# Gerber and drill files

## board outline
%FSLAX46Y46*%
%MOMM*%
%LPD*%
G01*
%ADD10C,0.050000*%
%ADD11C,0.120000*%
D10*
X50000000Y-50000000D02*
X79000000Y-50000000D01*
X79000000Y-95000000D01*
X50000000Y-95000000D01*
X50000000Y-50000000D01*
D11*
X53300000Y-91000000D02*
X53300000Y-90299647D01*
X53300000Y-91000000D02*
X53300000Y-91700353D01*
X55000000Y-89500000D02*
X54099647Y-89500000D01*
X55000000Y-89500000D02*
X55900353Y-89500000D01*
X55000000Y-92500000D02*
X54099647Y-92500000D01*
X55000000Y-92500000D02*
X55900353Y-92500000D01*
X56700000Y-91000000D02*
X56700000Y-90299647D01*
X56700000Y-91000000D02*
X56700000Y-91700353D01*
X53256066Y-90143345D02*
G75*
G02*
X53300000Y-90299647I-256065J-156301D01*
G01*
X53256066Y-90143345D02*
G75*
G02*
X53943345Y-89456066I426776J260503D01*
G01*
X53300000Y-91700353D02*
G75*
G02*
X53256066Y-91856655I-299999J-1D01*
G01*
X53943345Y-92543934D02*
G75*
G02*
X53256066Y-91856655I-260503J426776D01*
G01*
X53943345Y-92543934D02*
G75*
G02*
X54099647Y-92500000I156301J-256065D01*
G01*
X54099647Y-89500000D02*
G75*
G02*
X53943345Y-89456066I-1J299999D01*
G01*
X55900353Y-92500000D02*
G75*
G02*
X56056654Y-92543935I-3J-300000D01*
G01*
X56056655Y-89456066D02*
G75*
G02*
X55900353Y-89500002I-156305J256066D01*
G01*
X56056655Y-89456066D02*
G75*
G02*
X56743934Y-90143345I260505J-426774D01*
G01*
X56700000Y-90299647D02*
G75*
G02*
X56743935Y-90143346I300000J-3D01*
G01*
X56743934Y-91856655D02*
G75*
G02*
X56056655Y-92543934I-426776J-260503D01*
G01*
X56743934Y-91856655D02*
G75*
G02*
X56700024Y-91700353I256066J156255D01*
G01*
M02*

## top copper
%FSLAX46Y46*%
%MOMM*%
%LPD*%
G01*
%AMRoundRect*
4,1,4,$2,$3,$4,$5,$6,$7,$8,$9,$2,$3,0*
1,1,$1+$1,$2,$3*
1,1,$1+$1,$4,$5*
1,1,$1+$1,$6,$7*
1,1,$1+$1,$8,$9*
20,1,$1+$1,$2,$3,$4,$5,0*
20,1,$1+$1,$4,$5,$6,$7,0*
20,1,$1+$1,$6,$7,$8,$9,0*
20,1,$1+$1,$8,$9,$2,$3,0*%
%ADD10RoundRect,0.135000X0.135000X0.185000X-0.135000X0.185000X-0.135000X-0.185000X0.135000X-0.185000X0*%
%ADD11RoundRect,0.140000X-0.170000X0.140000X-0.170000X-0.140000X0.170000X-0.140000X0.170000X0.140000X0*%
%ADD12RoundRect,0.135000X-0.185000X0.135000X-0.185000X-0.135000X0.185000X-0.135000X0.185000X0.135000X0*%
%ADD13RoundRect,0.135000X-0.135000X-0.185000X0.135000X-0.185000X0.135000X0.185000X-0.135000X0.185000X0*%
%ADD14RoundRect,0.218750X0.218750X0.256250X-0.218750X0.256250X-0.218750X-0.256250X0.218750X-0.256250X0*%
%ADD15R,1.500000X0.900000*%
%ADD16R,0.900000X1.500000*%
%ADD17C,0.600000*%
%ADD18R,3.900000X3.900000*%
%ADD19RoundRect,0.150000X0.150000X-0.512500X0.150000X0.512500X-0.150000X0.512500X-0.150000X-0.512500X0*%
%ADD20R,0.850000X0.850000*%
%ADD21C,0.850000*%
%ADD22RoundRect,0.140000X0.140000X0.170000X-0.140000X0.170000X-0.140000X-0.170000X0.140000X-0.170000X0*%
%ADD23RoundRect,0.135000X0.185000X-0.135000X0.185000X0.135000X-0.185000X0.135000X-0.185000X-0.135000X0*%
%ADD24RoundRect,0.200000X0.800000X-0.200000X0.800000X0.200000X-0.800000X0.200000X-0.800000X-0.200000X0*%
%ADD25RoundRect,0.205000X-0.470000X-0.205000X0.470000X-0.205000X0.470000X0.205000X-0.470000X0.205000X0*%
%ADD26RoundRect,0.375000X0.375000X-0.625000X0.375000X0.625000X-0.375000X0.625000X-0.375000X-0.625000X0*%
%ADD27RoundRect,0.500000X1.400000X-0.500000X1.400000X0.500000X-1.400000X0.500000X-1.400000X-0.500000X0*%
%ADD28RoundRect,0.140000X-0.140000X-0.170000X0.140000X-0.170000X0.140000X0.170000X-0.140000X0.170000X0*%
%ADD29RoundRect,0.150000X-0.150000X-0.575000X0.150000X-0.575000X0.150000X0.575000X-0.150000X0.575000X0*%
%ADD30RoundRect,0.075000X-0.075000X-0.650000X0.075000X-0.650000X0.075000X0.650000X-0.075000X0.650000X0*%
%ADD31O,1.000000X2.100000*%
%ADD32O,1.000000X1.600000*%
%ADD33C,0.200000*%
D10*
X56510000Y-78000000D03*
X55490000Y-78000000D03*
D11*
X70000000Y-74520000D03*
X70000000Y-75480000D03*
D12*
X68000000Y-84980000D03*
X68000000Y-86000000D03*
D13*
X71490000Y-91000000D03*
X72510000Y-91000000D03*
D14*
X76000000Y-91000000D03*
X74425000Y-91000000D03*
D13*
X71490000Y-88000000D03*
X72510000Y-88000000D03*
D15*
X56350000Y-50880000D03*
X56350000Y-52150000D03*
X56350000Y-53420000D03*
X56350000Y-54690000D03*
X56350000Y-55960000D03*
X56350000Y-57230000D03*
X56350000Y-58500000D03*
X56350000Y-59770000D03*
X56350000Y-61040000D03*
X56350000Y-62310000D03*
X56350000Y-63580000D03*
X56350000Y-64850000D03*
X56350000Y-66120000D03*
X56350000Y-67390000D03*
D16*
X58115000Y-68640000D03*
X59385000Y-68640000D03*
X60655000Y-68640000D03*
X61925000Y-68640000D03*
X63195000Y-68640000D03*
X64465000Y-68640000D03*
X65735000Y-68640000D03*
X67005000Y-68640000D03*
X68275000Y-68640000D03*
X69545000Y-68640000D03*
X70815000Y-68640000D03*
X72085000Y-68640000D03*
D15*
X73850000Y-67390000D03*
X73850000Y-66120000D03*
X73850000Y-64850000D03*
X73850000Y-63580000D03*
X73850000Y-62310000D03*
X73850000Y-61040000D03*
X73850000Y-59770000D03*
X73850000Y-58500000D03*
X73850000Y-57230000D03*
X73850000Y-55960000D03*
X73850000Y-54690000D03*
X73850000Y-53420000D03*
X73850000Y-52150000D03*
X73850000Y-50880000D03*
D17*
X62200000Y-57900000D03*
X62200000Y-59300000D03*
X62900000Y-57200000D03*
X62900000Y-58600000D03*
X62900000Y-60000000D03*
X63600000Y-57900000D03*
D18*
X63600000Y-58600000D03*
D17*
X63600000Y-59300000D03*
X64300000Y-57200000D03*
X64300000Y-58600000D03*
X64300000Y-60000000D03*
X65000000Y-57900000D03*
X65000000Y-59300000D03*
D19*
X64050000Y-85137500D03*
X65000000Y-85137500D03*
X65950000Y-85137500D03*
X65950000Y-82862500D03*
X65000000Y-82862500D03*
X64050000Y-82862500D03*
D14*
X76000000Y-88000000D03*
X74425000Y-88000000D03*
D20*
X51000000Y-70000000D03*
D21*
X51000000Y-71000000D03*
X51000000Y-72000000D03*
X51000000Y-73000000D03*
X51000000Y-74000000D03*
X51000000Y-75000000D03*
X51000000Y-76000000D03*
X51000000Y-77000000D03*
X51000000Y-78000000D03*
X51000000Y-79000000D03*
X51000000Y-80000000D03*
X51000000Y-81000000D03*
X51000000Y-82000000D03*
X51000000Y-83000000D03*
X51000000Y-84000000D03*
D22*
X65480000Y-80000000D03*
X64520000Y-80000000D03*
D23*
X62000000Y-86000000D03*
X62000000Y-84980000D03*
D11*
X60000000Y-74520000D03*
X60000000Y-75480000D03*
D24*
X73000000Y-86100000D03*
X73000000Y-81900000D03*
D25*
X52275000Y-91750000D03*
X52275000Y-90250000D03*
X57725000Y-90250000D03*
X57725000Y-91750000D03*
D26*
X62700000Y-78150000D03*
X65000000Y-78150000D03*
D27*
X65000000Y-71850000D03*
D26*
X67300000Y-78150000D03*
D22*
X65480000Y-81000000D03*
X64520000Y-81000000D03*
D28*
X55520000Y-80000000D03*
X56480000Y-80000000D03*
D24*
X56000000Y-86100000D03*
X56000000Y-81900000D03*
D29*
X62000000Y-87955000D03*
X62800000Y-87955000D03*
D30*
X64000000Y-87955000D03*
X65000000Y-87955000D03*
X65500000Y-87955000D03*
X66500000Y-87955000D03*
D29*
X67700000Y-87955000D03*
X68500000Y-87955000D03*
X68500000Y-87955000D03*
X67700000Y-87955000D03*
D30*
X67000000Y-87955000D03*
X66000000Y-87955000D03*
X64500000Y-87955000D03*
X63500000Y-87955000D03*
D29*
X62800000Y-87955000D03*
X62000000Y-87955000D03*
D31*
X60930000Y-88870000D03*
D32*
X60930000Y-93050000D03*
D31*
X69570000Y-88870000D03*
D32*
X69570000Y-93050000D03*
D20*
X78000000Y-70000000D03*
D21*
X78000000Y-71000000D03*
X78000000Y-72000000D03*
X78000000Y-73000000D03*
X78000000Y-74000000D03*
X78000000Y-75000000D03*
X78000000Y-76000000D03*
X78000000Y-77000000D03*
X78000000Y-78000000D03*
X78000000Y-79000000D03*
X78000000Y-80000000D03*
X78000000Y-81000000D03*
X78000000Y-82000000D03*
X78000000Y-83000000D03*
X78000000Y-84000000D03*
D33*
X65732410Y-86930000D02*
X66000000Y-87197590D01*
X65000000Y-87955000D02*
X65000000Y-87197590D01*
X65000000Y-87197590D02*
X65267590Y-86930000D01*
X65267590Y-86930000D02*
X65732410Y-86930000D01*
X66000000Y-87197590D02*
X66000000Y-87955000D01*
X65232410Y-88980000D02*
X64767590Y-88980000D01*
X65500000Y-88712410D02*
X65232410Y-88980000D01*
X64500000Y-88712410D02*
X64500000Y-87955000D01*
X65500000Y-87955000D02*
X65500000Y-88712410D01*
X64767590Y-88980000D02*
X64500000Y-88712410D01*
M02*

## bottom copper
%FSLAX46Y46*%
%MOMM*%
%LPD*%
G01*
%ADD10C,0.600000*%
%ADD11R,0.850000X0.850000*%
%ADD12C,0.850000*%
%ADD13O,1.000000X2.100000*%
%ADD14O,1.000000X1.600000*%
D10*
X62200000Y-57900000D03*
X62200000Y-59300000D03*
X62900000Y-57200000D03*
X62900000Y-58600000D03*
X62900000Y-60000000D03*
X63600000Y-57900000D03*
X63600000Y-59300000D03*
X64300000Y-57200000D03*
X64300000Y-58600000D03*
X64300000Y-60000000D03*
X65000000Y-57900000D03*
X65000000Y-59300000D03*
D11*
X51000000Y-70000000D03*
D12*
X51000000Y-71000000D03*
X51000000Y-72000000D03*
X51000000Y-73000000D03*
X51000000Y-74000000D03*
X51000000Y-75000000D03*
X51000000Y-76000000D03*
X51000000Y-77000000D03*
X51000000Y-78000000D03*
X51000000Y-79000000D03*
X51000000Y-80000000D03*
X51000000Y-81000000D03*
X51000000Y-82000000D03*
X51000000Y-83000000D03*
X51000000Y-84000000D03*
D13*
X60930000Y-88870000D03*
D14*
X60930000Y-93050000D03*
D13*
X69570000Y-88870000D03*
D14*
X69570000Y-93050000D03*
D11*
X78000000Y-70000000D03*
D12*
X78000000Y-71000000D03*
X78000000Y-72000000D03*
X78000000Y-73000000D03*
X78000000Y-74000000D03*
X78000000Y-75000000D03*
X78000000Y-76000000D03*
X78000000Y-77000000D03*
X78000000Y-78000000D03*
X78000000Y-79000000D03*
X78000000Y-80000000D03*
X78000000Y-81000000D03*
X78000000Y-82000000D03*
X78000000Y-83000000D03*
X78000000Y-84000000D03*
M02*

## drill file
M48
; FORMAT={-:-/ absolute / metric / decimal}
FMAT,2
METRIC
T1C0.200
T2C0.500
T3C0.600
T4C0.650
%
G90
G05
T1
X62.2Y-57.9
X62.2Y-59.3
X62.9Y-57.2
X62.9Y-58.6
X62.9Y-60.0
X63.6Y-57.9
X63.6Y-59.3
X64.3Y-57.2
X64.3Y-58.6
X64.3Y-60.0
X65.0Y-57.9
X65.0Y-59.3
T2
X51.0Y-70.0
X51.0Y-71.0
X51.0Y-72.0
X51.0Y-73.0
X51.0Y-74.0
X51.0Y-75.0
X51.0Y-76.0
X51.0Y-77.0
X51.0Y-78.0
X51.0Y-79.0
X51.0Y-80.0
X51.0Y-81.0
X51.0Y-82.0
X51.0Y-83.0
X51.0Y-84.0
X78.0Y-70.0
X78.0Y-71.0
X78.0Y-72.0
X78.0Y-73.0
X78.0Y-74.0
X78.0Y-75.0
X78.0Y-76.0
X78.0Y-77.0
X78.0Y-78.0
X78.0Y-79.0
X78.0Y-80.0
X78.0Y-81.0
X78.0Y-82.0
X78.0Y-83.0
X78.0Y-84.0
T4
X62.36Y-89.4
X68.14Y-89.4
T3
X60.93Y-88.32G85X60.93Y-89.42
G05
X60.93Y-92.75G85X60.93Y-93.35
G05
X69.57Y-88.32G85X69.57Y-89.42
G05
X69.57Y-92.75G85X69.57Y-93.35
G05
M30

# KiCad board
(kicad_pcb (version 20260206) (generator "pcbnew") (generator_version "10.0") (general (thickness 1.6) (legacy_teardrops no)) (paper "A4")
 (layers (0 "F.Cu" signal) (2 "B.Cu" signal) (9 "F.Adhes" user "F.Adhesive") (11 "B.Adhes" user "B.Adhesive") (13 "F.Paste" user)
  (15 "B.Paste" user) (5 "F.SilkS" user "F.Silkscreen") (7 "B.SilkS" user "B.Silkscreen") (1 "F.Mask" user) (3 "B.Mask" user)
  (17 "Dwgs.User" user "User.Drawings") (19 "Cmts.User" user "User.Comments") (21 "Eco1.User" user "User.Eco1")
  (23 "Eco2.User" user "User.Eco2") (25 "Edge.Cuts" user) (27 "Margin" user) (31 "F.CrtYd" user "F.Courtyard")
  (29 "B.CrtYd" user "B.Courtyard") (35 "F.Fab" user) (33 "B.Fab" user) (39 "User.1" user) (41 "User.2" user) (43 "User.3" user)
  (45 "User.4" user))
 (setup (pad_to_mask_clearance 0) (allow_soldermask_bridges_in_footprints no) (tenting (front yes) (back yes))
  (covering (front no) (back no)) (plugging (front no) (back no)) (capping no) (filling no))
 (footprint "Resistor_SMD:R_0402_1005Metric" (layer "F.Cu") (at 56 78 180)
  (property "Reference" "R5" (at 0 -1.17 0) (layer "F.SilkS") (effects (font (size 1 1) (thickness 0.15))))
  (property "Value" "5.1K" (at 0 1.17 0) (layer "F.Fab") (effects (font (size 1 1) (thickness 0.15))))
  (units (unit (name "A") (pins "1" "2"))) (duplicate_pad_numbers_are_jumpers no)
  (pad "1" smd roundrect (at -0.51 0 180) (size 0.54 0.64) (layers "F.Cu" "F.Mask" "F.Paste") (roundrect_rratio 0.25) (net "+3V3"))
  (pad "2" smd roundrect (at 0.51 0 180) (size 0.54 0.64) (layers "F.Cu" "F.Mask" "F.Paste") (roundrect_rratio 0.25) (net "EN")))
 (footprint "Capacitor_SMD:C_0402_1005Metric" (layer "F.Cu") (at 70 75 -90)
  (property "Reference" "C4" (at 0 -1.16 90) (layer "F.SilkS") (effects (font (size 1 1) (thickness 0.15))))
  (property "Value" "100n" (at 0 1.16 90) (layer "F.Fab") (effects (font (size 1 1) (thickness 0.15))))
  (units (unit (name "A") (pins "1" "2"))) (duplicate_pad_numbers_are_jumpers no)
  (pad "1" smd roundrect (at -0.48 0 270) (size 0.56 0.62) (layers "F.Cu" "F.Mask" "F.Paste") (roundrect_rratio 0.25) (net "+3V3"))
  (pad "2" smd roundrect (at 0.48 0 270) (size 0.56 0.62) (layers "F.Cu" "F.Mask" "F.Paste") (roundrect_rratio 0.25) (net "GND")))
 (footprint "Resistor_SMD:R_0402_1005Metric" (layer "F.Cu") (at 68 85.49 -90)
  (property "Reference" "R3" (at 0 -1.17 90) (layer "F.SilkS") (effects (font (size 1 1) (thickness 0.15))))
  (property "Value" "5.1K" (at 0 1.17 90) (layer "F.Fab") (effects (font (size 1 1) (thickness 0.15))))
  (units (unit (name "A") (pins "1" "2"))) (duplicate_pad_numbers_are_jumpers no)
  (pad "1" smd roundrect (at -0.51 0 270) (size 0.54 0.64) (layers "F.Cu" "F.Mask" "F.Paste") (roundrect_rratio 0.25) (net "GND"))
  (pad "2" smd roundrect (at 0.51 0 270) (size 0.54 0.64) (layers "F.Cu" "F.Mask" "F.Paste") (roundrect_rratio 0.25) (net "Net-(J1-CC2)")))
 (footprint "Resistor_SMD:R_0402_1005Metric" (layer "F.Cu") (at 72 91)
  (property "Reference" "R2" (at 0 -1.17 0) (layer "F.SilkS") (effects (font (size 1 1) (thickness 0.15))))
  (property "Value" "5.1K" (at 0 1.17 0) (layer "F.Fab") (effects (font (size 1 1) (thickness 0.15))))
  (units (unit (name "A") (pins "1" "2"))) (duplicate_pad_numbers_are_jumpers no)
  (pad "1" smd roundrect (at -0.51 0) (size 0.54 0.64) (layers "F.Cu" "F.Mask" "F.Paste") (roundrect_rratio 0.25) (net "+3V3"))
  (pad "2" smd roundrect (at 0.51 0) (size 0.54 0.64) (layers "F.Cu" "F.Mask" "F.Paste") (roundrect_rratio 0.25) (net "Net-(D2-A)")))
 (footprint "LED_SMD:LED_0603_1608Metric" (layer "F.Cu") (at 75.2125 91 180)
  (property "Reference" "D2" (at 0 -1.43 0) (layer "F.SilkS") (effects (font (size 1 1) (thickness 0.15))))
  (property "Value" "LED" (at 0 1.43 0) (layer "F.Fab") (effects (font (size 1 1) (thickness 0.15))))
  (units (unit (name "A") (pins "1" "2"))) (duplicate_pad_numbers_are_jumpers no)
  (pad "1" smd roundrect (at -0.7875 0 180) (size 0.875 0.95) (layers "F.Cu" "F.Mask" "F.Paste") (roundrect_rratio 0.25) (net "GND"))
  (pad "2" smd roundrect (at 0.7875 0 180) (size 0.875 0.95) (layers "F.Cu" "F.Mask" "F.Paste") (roundrect_rratio 0.25) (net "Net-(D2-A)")))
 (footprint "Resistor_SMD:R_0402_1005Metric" (layer "F.Cu") (at 72 88)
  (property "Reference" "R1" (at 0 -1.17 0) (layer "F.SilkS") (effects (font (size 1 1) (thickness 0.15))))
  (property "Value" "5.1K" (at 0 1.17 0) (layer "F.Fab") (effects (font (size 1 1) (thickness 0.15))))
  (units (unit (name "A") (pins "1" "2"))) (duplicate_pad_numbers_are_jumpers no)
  (pad "1" smd roundrect (at -0.51 0) (size 0.54 0.64) (layers "F.Cu" "F.Mask" "F.Paste") (roundrect_rratio 0.25) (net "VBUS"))
  (pad "2" smd roundrect (at 0.51 0) (size 0.54 0.64) (layers "F.Cu" "F.Mask" "F.Paste") (roundrect_rratio 0.25) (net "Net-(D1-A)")))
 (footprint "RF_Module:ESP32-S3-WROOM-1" (layer "F.Cu") (at 65.1 56.14)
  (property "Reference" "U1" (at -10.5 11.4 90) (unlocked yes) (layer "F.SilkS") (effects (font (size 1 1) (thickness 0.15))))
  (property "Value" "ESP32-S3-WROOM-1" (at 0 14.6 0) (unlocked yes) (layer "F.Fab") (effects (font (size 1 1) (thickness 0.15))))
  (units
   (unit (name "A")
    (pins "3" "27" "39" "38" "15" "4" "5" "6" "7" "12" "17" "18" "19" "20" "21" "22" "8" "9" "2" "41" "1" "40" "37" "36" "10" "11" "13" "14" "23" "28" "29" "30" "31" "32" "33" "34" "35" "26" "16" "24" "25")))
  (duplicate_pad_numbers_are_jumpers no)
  (pad "" smd rect (at -2.9 1.06) (size 0.9 0.9) (layers "F.Paste"))
  (pad "" smd rect (at -2.9 2.46 270) (size 0.9 0.9) (layers "F.Paste"))
  (pad "" smd rect (at -2.9 3.86) (size 0.9 0.9) (layers "F.Paste"))
  (pad "" smd rect (at -1.5 1.06 270) (size 0.9 0.9) (layers "F.Paste"))
  (pad "" smd rect (at -1.5 2.46 270) (size 0.9 0.9) (layers "F.Paste"))
  (pad "" smd rect (at -1.5 3.86 270) (size 0.9 0.9) (layers "F.Paste"))
  (pad "" smd rect (at -0.1 1.06 270) (size 0.9 0.9) (layers "F.Paste"))
  (pad "" smd rect (at -0.1 2.46 270) (size 0.9 0.9) (layers "F.Paste"))
  (pad "" smd rect (at -0.1 3.86 270) (size 0.9 0.9) (layers "F.Paste"))
  (pad "1" smd rect (at -8.75 -5.26) (size 1.5 0.9) (layers "F.Cu" "F.Mask" "F.Paste") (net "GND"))
  (pad "2" smd rect (at -8.75 -3.99) (size 1.5 0.9) (layers "F.Cu" "F.Mask" "F.Paste") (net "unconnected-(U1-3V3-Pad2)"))
  (pad "3" smd rect (at -8.75 -2.72) (size 1.5 0.9) (layers "F.Cu" "F.Mask" "F.Paste") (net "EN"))
  (pad "4" smd rect (at -8.75 -1.45) (size 1.5 0.9) (layers "F.Cu" "F.Mask" "F.Paste") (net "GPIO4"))
  (pad "5" smd rect (at -8.75 -0.18) (size 1.5 0.9) (layers "F.Cu" "F.Mask" "F.Paste") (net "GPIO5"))
  (pad "6" smd rect (at -8.75 1.09) (size 1.5 0.9) (layers "F.Cu" "F.Mask" "F.Paste") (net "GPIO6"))
  (pad "7" smd rect (at -8.75 2.36) (size 1.5 0.9) (layers "F.Cu" "F.Mask" "F.Paste") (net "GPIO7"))
  (pad "8" smd rect (at -8.75 3.63) (size 1.5 0.9) (layers "F.Cu" "F.Mask" "F.Paste") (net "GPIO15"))
  (pad "9" smd rect (at -8.75 4.9) (size 1.5 0.9) (layers "F.Cu" "F.Mask" "F.Paste") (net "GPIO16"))
  (pad "10" smd rect (at -8.75 6.17) (size 1.5 0.9) (layers "F.Cu" "F.Mask" "F.Paste") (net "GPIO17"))
  (pad "11" smd rect (at -8.75 7.44) (size 1.5 0.9) (layers "F.Cu" "F.Mask" "F.Paste") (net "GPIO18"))
  (pad "12" smd rect (at -8.75 8.71) (size 1.5 0.9) (layers "F.Cu" "F.Mask" "F.Paste") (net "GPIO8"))
  (pad "13" smd rect (at -8.75 9.98) (size 1.5 0.9) (layers "F.Cu" "F.Mask" "F.Paste") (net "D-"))
  (pad "14" smd rect (at -8.75 11.25 180) (size 1.5 0.9) (layers "F.Cu" "F.Mask" "F.Paste") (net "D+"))
  (pad "15" smd rect (at -6.985 12.5 270) (size 1.5 0.9) (layers "F.Cu" "F.Mask" "F.Paste") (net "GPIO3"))
  (pad "16" smd rect (at -5.715 12.5 270) (size 1.5 0.9) (layers "F.Cu" "F.Mask" "F.Paste") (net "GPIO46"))
  (pad "17" smd rect (at -4.445 12.5 270) (size 1.5 0.9) (layers "F.Cu" "F.Mask" "F.Paste") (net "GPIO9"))
  (pad "18" smd rect (at -3.175 12.5 270) (size 1.5 0.9) (layers "F.Cu" "F.Mask" "F.Paste") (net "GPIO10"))
  (pad "19" smd rect (at -1.905 12.5 270) (size 1.5 0.9) (layers "F.Cu" "F.Mask" "F.Paste") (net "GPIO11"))
  (pad "20" smd rect (at -0.635 12.5 270) (size 1.5 0.9) (layers "F.Cu" "F.Mask" "F.Paste") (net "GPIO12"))
  (pad "21" smd rect (at 0.635 12.5 270) (size 1.5 0.9) (layers "F.Cu" "F.Mask" "F.Paste") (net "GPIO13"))
  (pad "22" smd rect (at 1.905 12.5 270) (size 1.5 0.9) (layers "F.Cu" "F.Mask" "F.Paste") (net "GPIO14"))
  (pad "23" smd rect (at 3.175 12.5 270) (size 1.5 0.9) (layers "F.Cu" "F.Mask" "F.Paste") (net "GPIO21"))
  (pad "24" smd rect (at 4.445 12.5 270) (size 1.5 0.9) (layers "F.Cu" "F.Mask" "F.Paste") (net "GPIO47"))
  (pad "25" smd rect (at 5.715 12.5 270) (size 1.5 0.9) (layers "F.Cu" "F.Mask" "F.Paste") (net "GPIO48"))
  (pad "26" smd rect (at 6.985 12.5 270) (size 1.5 0.9) (layers "F.Cu" "F.Mask" "F.Paste") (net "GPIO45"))
  (pad "27" smd rect (at 8.75 11.25) (size 1.5 0.9) (layers "F.Cu" "F.Mask" "F.Paste") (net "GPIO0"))
  (pad "28" smd rect (at 8.75 9.98) (size 1.5 0.9) (layers "F.Cu" "F.Mask" "F.Paste") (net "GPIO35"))
  (pad "29" smd rect (at 8.75 8.71) (size 1.5 0.9) (layers "F.Cu" "F.Mask" "F.Paste") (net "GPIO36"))
  (pad "30" smd rect (at 8.75 7.44) (size 1.5 0.9) (layers "F.Cu" "F.Mask" "F.Paste") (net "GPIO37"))
  (pad "31" smd rect (at 8.75 6.17) (size 1.5 0.9) (layers "F.Cu" "F.Mask" "F.Paste") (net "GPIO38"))
  (pad "32" smd rect (at 8.75 4.9) (size 1.5 0.9) (layers "F.Cu" "F.Mask" "F.Paste") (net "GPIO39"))
  (pad "33" smd rect (at 8.75 3.63) (size 1.5 0.9) (layers "F.Cu" "F.Mask" "F.Paste") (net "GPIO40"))
  (pad "34" smd rect (at 8.75 2.36) (size 1.5 0.9) (layers "F.Cu" "F.Mask" "F.Paste") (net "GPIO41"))
  (pad "35" smd rect (at 8.75 1.09) (size 1.5 0.9) (layers "F.Cu" "F.Mask" "F.Paste") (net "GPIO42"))
  (pad "36" smd rect (at 8.75 -0.18) (size 1.5 0.9) (layers "F.Cu" "F.Mask" "F.Paste") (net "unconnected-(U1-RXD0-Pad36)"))
  (pad "37" smd rect (at 8.75 -1.45) (size 1.5 0.9) (layers "F.Cu" "F.Mask" "F.Paste") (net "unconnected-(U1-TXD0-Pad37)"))
  (pad "38" smd rect (at 8.75 -2.72) (size 1.5 0.9) (layers "F.Cu" "F.Mask" "F.Paste") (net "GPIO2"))
  (pad "39" smd rect (at 8.75 -3.99) (size 1.5 0.9) (layers "F.Cu" "F.Mask" "F.Paste") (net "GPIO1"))
  (pad "40" smd rect (at 8.75 -5.26) (size 1.5 0.9) (layers "F.Cu" "F.Mask" "F.Paste") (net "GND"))
  (pad "41" thru_hole circle (at -2.9 1.76 90) (size 0.6 0.6) (drill 0.2) (layers "*.Cu" "F.Mask") (remove_unused_layers no) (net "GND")
   (zone_connect 2))
  (pad "41" thru_hole circle (at -2.9 3.16) (size 0.6 0.6) (drill 0.2) (layers "*.Cu" "F.Mask") (remove_unused_layers no) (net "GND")
   (zone_connect 2))
  (pad "41" thru_hole circle (at -2.2 1.06) (size 0.6 0.6) (drill 0.2) (layers "*.Cu" "F.Mask") (remove_unused_layers no) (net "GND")
   (zone_connect 2))
  (pad "41" thru_hole circle (at -2.2 2.46) (size 0.6 0.6) (drill 0.2) (layers "*.Cu" "F.Mask") (remove_unused_layers no) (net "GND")
   (zone_connect 2))
  (pad "41" thru_hole circle (at -2.2 3.86) (size 0.6 0.6) (drill 0.2) (layers "*.Cu" "F.Mask") (remove_unused_layers no) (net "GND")
   (zone_connect 2))
  (pad "41" thru_hole circle (at -1.5 1.76) (size 0.6 0.6) (drill 0.2) (layers "*.Cu" "F.Mask") (remove_unused_layers no) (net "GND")
   (zone_connect 2))
  (pad "41" smd rect (at -1.5 2.46 270) (size 3.9 3.9) (layers "F.Cu" "F.Mask") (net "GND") (zone_connect 2))
  (pad "41" thru_hole circle (at -1.5 3.16) (size 0.6 0.6) (drill 0.2) (layers "*.Cu" "F.Mask") (remove_unused_layers no) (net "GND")
   (zone_connect 2))
  (pad "41" thru_hole circle (at -0.8 1.06) (size 0.6 0.6) (drill 0.2) (layers "*.Cu" "F.Mask") (remove_unused_layers no) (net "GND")
   (zone_connect 2))
  (pad "41" thru_hole circle (at -0.8 2.46) (size 0.6 0.6) (drill 0.2) (layers "*.Cu" "F.Mask") (remove_unused_layers no) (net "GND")
   (zone_connect 2))
  (pad "41" thru_hole circle (at -0.8 3.86) (size 0.6 0.6) (drill 0.2) (layers "*.Cu" "F.Mask") (remove_unused_layers no) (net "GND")
   (zone_connect 2))
  (pad "41" thru_hole circle (at -0.1 1.76) (size 0.6 0.6) (drill 0.2) (layers "*.Cu" "F.Mask") (remove_unused_layers no) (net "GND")
   (zone_connect 2))
  (pad "41" thru_hole circle (at -0.1 3.16) (size 0.6 0.6) (drill 0.2) (layers "*.Cu" "F.Mask") (remove_unused_layers no) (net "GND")
   (zone_connect 2))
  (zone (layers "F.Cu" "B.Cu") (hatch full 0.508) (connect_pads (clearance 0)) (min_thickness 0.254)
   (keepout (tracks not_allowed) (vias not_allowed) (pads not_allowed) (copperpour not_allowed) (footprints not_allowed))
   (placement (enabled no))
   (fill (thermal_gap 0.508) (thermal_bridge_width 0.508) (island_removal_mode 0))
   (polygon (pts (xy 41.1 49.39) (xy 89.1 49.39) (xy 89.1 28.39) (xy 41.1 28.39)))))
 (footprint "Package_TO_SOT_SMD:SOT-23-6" (layer "F.Cu") (at 65 84 90)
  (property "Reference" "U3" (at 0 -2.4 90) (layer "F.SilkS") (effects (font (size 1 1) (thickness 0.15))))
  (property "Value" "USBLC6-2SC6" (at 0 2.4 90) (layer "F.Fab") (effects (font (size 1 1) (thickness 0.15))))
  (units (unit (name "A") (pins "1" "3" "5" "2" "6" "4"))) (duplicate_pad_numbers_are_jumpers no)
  (pad "1" smd roundrect (at -1.1375 -0.95 90) (size 1.325 0.6) (layers "F.Cu" "F.Mask" "F.Paste") (roundrect_rratio 0.25)
   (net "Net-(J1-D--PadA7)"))
  (pad "2" smd roundrect (at -1.1375 0 90) (size 1.325 0.6) (layers "F.Cu" "F.Mask" "F.Paste") (roundrect_rratio 0.25) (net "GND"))
  (pad "3" smd roundrect (at -1.1375 0.95 90) (size 1.325 0.6) (layers "F.Cu" "F.Mask" "F.Paste") (roundrect_rratio 0.25)
   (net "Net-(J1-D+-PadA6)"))
  (pad "4" smd roundrect (at 1.1375 0.95 90) (size 1.325 0.6) (layers "F.Cu" "F.Mask" "F.Paste") (roundrect_rratio 0.25) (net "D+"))
  (pad "5" smd roundrect (at 1.1375 0 90) (size 1.325 0.6) (layers "F.Cu" "F.Mask" "F.Paste") (roundrect_rratio 0.25) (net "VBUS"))
  (pad "6" smd roundrect (at 1.1375 -0.95 90) (size 1.325 0.6) (layers "F.Cu" "F.Mask" "F.Paste") (roundrect_rratio 0.25) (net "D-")))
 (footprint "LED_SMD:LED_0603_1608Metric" (layer "F.Cu") (at 75.2125 88 180)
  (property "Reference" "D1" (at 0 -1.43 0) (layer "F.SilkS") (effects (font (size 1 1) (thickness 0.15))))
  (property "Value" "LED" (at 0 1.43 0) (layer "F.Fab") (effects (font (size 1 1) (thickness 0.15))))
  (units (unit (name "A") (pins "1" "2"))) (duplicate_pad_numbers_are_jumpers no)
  (pad "1" smd roundrect (at -0.7875 0 180) (size 0.875 0.95) (layers "F.Cu" "F.Mask" "F.Paste") (roundrect_rratio 0.25) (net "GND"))
  (pad "2" smd roundrect (at 0.7875 0 180) (size 0.875 0.95) (layers "F.Cu" "F.Mask" "F.Paste") (roundrect_rratio 0.25) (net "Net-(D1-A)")))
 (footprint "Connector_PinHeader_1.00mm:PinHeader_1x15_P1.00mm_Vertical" (layer "F.Cu") (at 51 70)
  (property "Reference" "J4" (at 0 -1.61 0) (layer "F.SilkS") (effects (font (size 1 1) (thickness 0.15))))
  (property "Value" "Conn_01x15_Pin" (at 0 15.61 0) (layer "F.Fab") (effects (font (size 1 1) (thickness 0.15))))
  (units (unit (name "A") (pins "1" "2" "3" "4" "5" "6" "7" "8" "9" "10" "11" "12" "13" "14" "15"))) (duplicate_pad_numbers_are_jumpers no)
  (pad "1" thru_hole rect (at 0 0) (size 0.85 0.85) (drill 0.5) (layers "*.Cu" "*.Mask") (remove_unused_layers no) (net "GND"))
  (pad "2" thru_hole circle (at 0 1) (size 0.85 0.85) (drill 0.5) (layers "*.Cu" "*.Mask") (remove_unused_layers no) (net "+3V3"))
  (pad "3" thru_hole circle (at 0 2) (size 0.85 0.85) (drill 0.5) (layers "*.Cu" "*.Mask") (remove_unused_layers no) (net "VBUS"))
  (pad "4" thru_hole circle (at 0 3) (size 0.85 0.85) (drill 0.5) (layers "*.Cu" "*.Mask") (remove_unused_layers no) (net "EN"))
  (pad "5" thru_hole circle (at 0 4) (size 0.85 0.85) (drill 0.5) (layers "*.Cu" "*.Mask") (remove_unused_layers no) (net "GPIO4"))
  (pad "6" thru_hole circle (at 0 5) (size 0.85 0.85) (drill 0.5) (layers "*.Cu" "*.Mask") (remove_unused_layers no) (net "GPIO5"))
  (pad "7" thru_hole circle (at 0 6) (size 0.85 0.85) (drill 0.5) (layers "*.Cu" "*.Mask") (remove_unused_layers no) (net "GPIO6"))
  (pad "8" thru_hole circle (at 0 7) (size 0.85 0.85) (drill 0.5) (layers "*.Cu" "*.Mask") (remove_unused_layers no) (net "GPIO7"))
  (pad "9" thru_hole circle (at 0 8) (size 0.85 0.85) (drill 0.5) (layers "*.Cu" "*.Mask") (remove_unused_layers no) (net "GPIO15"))
  (pad "10" thru_hole circle (at 0 9) (size 0.85 0.85) (drill 0.5) (layers "*.Cu" "*.Mask") (remove_unused_layers no) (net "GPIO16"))
  (pad "11" thru_hole circle (at 0 10) (size 0.85 0.85) (drill 0.5) (layers "*.Cu" "*.Mask") (remove_unused_layers no) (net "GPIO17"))
  (pad "12" thru_hole circle (at 0 11) (size 0.85 0.85) (drill 0.5) (layers "*.Cu" "*.Mask") (remove_unused_layers no) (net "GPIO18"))
  (pad "13" thru_hole circle (at 0 12) (size 0.85 0.85) (drill 0.5) (layers "*.Cu" "*.Mask") (remove_unused_layers no) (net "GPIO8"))
  (pad "14" thru_hole circle (at 0 13) (size 0.85 0.85) (drill 0.5) (layers "*.Cu" "*.Mask") (remove_unused_layers no) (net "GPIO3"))
  (pad "15" thru_hole circle (at 0 14) (size 0.85 0.85) (drill 0.5) (layers "*.Cu" "*.Mask") (remove_unused_layers no) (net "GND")))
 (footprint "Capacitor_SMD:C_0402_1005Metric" (layer "F.Cu") (at 65 80 180)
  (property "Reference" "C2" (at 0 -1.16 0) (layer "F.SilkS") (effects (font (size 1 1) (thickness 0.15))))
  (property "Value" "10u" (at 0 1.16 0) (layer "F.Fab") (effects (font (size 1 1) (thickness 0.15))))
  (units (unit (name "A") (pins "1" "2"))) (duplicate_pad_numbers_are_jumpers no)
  (pad "1" smd roundrect (at -0.48 0 180) (size 0.56 0.62) (layers "F.Cu" "F.Mask" "F.Paste") (roundrect_rratio 0.25) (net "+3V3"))
  (pad "2" smd roundrect (at 0.48 0 180) (size 0.56 0.62) (layers "F.Cu" "F.Mask" "F.Paste") (roundrect_rratio 0.25) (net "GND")))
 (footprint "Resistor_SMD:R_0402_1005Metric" (layer "F.Cu") (at 62 85.49 90)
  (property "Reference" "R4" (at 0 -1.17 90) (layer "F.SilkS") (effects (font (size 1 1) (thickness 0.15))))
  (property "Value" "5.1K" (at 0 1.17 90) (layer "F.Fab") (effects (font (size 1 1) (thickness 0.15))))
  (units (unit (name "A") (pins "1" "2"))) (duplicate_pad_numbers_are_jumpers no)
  (pad "1" smd roundrect (at -0.51 0 90) (size 0.54 0.64) (layers "F.Cu" "F.Mask" "F.Paste") (roundrect_rratio 0.25) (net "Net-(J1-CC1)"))
  (pad "2" smd roundrect (at 0.51 0 90) (size 0.54 0.64) (layers "F.Cu" "F.Mask" "F.Paste") (roundrect_rratio 0.25) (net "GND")))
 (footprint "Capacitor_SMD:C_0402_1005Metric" (layer "F.Cu") (at 60 75 -90)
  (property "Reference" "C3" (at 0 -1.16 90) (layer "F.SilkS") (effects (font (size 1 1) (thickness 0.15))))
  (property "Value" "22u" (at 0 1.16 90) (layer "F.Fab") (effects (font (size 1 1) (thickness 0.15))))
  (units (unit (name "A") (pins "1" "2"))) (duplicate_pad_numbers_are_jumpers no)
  (pad "1" smd roundrect (at -0.48 0 270) (size 0.56 0.62) (layers "F.Cu" "F.Mask" "F.Paste") (roundrect_rratio 0.25) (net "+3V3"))
  (pad "2" smd roundrect (at 0.48 0 270) (size 0.56 0.62) (layers "F.Cu" "F.Mask" "F.Paste") (roundrect_rratio 0.25) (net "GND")))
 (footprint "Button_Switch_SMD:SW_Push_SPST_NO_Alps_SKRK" (layer "F.Cu") (at 73 84 90)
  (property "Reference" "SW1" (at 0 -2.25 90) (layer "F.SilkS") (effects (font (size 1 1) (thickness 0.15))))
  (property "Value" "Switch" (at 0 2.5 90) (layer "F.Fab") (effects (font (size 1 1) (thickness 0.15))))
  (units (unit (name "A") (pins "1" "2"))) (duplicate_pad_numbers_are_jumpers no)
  (pad "1" smd roundrect (at -2.1 0 90) (size 0.8 2) (layers "F.Cu" "F.Mask" "F.Paste") (roundrect_rratio 0.25) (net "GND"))
  (pad "2" smd roundrect (at 2.1 0 90) (size 0.8 2) (layers "F.Cu" "F.Mask" "F.Paste") (roundrect_rratio 0.25) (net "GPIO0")))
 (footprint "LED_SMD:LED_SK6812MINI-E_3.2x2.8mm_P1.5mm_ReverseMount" (layer "F.Cu") (at 55 91)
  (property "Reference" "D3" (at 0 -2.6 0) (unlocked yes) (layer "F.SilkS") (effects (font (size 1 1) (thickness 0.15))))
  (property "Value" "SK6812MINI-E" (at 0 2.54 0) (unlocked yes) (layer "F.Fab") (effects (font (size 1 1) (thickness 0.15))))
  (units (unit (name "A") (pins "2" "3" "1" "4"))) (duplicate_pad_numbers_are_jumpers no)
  (fp_line (start -1.7 0) (end -1.7 -0.700353) (stroke (width 0.12) (type solid)) (layer "Edge.Cuts"))
  (fp_line (start -1.7 0) (end -1.7 0.700353) (stroke (width 0.12) (type solid)) (layer "Edge.Cuts"))
  (fp_line (start 0 -1.5) (end -0.900353 -1.5) (stroke (width 0.12) (type solid)) (layer "Edge.Cuts"))
  (fp_line (start 0 -1.5) (end 0.900353 -1.5) (stroke (width 0.12) (type solid)) (layer "Edge.Cuts"))
  (fp_line (start 0 1.5) (end -0.900353 1.5) (stroke (width 0.12) (type solid)) (layer "Edge.Cuts"))
  (fp_line (start 0 1.5) (end 0.900353 1.5) (stroke (width 0.12) (type solid)) (layer "Edge.Cuts"))
  (fp_line (start 1.7 0) (end 1.7 -0.700353) (stroke (width 0.12) (type solid)) (layer "Edge.Cuts"))
  (fp_line (start 1.7 0) (end 1.7 0.700353) (stroke (width 0.12) (type solid)) (layer "Edge.Cuts"))
  (fp_arc (start -1.743934 -0.856655) (mid -1.711192 -0.781532) (end -1.7 -0.700353) (stroke (width 0.12) (type solid)) (layer "Edge.Cuts"))
  (fp_arc (start -1.743934 -0.856655) (mid -1.670711 -1.470711) (end -1.056655 -1.543934) (stroke (width 0.12) (type solid))
   (layer "Edge.Cuts"))
  (fp_arc (start -1.7 0.700353) (mid -1.711192 0.781532) (end -1.743934 0.856655) (stroke (width 0.12) (type solid)) (layer "Edge.Cuts"))
  (fp_arc (start -1.056655 1.543934) (mid -1.670711 1.470711) (end -1.743934 0.856655) (stroke (width 0.12) (type solid))
   (layer "Edge.Cuts"))
  (fp_arc (start -1.056655 1.543934) (mid -0.981532 1.511192) (end -0.900353 1.5) (stroke (width 0.12) (type solid)) (layer "Edge.Cuts"))
  (fp_arc (start -0.900353 -1.5) (mid -0.981532 -1.511192) (end -1.056655 -1.543934) (stroke (width 0.12) (type solid)) (layer "Edge.Cuts"))
  (fp_arc (start 0.900353 1.5) (mid 0.981532 1.511192) (end 1.056655 1.543934) (stroke (width 0.12) (type solid)) (layer "Edge.Cuts"))
  (fp_arc (start 1.056655 -1.543934) (mid 0.981532 -1.511192) (end 0.900353 -1.5) (stroke (width 0.12) (type solid)) (layer "Edge.Cuts"))
  (fp_arc (start 1.056655 -1.543934) (mid 1.670711 -1.470711) (end 1.743934 -0.856655) (stroke (width 0.12) (type solid))
   (layer "Edge.Cuts"))
  (fp_arc (start 1.7 -0.700353) (mid 1.711192 -0.781532) (end 1.743934 -0.856655) (stroke (width 0.12) (type solid)) (layer "Edge.Cuts"))
  (fp_arc (start 1.743934 0.856655) (mid 1.670711 1.470711) (end 1.056655 1.543934) (stroke (width 0.12) (type solid)) (layer "Edge.Cuts"))
  (fp_arc (start 1.743934 0.856655) (mid 1.711192 0.781532) (end 1.7 0.700353) (stroke (width 0.12) (type solid)) (layer "Edge.Cuts"))
  (pad "1" smd roundrect (at -2.725 0.75) (size 1.35 0.82) (layers "F.Cu" "F.Mask" "F.Paste") (roundrect_rratio 0.25) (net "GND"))
  (pad "2" smd roundrect (at -2.725 -0.75) (size 1.35 0.82) (layers "F.Cu" "F.Mask" "F.Paste") (roundrect_rratio 0.25) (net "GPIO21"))
  (pad "3" smd roundrect (at 2.725 -0.75) (size 1.35 0.82) (layers "F.Cu" "F.Mask" "F.Paste") (roundrect_rratio 0.25) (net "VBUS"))
  (pad "4" smd roundrect (at 2.725 0.75) (size 1.35 0.82) (layers "F.Cu" "F.Mask" "F.Paste") (roundrect_rratio 0.25)
   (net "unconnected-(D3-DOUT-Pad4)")))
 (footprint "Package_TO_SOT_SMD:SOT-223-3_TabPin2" (layer "F.Cu") (at 65 75 90)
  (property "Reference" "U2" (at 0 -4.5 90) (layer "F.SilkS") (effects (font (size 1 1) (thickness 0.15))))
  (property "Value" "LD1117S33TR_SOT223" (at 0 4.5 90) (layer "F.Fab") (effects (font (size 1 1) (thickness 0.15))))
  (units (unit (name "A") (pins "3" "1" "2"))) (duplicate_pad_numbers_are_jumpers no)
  (pad "1" smd roundrect (at -3.15 -2.3 90) (size 2 1.5) (layers "F.Cu" "F.Mask" "F.Paste") (roundrect_rratio 0.25) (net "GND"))
  (pad "2" smd roundrect (at -3.15 0 90) (size 2 1.5) (layers "F.Cu" "F.Mask" "F.Paste") (roundrect_rratio 0.25) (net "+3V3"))
  (pad "2" smd roundrect (at 3.15 0 90) (size 2 3.8) (layers "F.Cu" "F.Mask" "F.Paste") (roundrect_rratio 0.25) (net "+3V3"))
  (pad "3" smd roundrect (at -3.15 2.3 90) (size 2 1.5) (layers "F.Cu" "F.Mask" "F.Paste") (roundrect_rratio 0.25) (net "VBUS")))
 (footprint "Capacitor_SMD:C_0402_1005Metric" (layer "F.Cu") (at 65 81 180)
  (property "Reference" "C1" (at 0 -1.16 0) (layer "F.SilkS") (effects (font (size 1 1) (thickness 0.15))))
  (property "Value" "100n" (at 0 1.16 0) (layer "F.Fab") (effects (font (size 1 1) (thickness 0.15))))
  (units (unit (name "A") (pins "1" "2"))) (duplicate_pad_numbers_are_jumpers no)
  (pad "1" smd roundrect (at -0.48 0 180) (size 0.56 0.62) (layers "F.Cu" "F.Mask" "F.Paste") (roundrect_rratio 0.25) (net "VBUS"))
  (pad "2" smd roundrect (at 0.48 0 180) (size 0.56 0.62) (layers "F.Cu" "F.Mask" "F.Paste") (roundrect_rratio 0.25) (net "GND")))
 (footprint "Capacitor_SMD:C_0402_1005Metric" (layer "F.Cu") (at 56 80)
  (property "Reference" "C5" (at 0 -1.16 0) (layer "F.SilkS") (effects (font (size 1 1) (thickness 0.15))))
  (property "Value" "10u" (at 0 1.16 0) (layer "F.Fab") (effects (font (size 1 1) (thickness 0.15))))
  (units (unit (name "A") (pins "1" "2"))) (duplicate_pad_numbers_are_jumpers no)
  (pad "1" smd roundrect (at -0.48 0) (size 0.56 0.62) (layers "F.Cu" "F.Mask" "F.Paste") (roundrect_rratio 0.25) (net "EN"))
  (pad "2" smd roundrect (at 0.48 0) (size 0.56 0.62) (layers "F.Cu" "F.Mask" "F.Paste") (roundrect_rratio 0.25) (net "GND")))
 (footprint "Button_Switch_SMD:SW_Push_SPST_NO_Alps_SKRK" (layer "F.Cu") (at 56 84 90)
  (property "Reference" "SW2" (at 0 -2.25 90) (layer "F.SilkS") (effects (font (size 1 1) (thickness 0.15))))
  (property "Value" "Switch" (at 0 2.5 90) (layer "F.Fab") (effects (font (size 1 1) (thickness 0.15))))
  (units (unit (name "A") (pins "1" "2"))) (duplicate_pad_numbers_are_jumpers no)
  (pad "1" smd roundrect (at -2.1 0 90) (size 0.8 2) (layers "F.Cu" "F.Mask" "F.Paste") (roundrect_rratio 0.25) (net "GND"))
  (pad "2" smd roundrect (at 2.1 0 90) (size 0.8 2) (layers "F.Cu" "F.Mask" "F.Paste") (roundrect_rratio 0.25) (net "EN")))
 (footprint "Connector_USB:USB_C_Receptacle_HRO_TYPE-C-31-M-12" (layer "F.Cu") (at 65.25 92)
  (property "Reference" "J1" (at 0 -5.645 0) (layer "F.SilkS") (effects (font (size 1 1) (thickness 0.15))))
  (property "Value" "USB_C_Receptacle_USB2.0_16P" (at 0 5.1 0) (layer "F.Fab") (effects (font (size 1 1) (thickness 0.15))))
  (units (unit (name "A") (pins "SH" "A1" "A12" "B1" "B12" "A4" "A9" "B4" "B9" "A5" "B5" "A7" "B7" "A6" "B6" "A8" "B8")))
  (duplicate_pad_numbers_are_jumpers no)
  (pad "" np_thru_hole circle (at -2.89 -2.6) (size 0.65 0.65) (drill 0.65) (layers "*.Cu" "*.Mask"))
  (pad "" np_thru_hole circle (at 2.89 -2.6) (size 0.65 0.65) (drill 0.65) (layers "*.Cu" "*.Mask"))
  (pad "A1" smd roundrect (at -3.25 -4.045) (size 0.6 1.45) (layers "F.Cu" "F.Mask" "F.Paste") (roundrect_rratio 0.25) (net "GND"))
  (pad "A4" smd roundrect (at -2.45 -4.045) (size 0.6 1.45) (layers "F.Cu" "F.Mask" "F.Paste") (roundrect_rratio 0.25) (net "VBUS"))
  (pad "A5" smd roundrect (at -1.25 -4.045) (size 0.3 1.45) (layers "F.Cu" "F.Mask" "F.Paste") (roundrect_rratio 0.25) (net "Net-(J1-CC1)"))
  (pad "A6" smd roundrect (at -0.25 -4.045) (size 0.3 1.45) (layers "F.Cu" "F.Mask" "F.Paste") (roundrect_rratio 0.25)
   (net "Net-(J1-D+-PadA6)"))
  (pad "A7" smd roundrect (at 0.25 -4.045) (size 0.3 1.45) (layers "F.Cu" "F.Mask" "F.Paste") (roundrect_rratio 0.25)
   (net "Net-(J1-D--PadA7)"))
  (pad "A8" smd roundrect (at 1.25 -4.045) (size 0.3 1.45) (layers "F.Cu" "F.Mask" "F.Paste") (roundrect_rratio 0.25)
   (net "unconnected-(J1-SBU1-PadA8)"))
  (pad "A9" smd roundrect (at 2.45 -4.045) (size 0.6 1.45) (layers "F.Cu" "F.Mask" "F.Paste") (roundrect_rratio 0.25) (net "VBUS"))
  (pad "A12" smd roundrect (at 3.25 -4.045) (size 0.6 1.45) (layers "F.Cu" "F.Mask" "F.Paste") (roundrect_rratio 0.25) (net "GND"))
  (pad "B1" smd roundrect (at 3.25 -4.045) (size 0.6 1.45) (layers "F.Cu" "F.Mask" "F.Paste") (roundrect_rratio 0.25) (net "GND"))
  (pad "B4" smd roundrect (at 2.45 -4.045) (size 0.6 1.45) (layers "F.Cu" "F.Mask" "F.Paste") (roundrect_rratio 0.25) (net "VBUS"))
  (pad "B5" smd roundrect (at 1.75 -4.045) (size 0.3 1.45) (layers "F.Cu" "F.Mask" "F.Paste") (roundrect_rratio 0.25) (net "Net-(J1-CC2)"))
  (pad "B6" smd roundrect (at 0.75 -4.045) (size 0.3 1.45) (layers "F.Cu" "F.Mask" "F.Paste") (roundrect_rratio 0.25)
   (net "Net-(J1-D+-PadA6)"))
  (pad "B7" smd roundrect (at -0.75 -4.045) (size 0.3 1.45) (layers "F.Cu" "F.Mask" "F.Paste") (roundrect_rratio 0.25)
   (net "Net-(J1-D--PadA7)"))
  (pad "B8" smd roundrect (at -1.75 -4.045) (size 0.3 1.45) (layers "F.Cu" "F.Mask" "F.Paste") (roundrect_rratio 0.25)
   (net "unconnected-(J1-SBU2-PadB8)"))
  (pad "B9" smd roundrect (at -2.45 -4.045) (size 0.6 1.45) (layers "F.Cu" "F.Mask" "F.Paste") (roundrect_rratio 0.25) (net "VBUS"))
  (pad "B12" smd roundrect (at -3.25 -4.045) (size 0.6 1.45) (layers "F.Cu" "F.Mask" "F.Paste") (roundrect_rratio 0.25) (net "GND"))
  (pad "SH" thru_hole oval (at -4.32 -3.13) (size 1 2.1) (drill oval 0.6 1.7) (layers "*.Cu" "*.Mask") (remove_unused_layers no) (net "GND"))
  (pad "SH" thru_hole oval (at -4.32 1.05) (size 1 1.6) (drill oval 0.6 1.2) (layers "*.Cu" "*.Mask") (remove_unused_layers no) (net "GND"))
  (pad "SH" thru_hole oval (at 4.32 -3.13) (size 1 2.1) (drill oval 0.6 1.7) (layers "*.Cu" "*.Mask") (remove_unused_layers no) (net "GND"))
  (pad "SH" thru_hole oval (at 4.32 1.05) (size 1 1.6) (drill oval 0.6 1.2) (layers "*.Cu" "*.Mask") (remove_unused_layers no) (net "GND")))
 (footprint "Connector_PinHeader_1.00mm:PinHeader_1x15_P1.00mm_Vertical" (layer "F.Cu") (at 78 70)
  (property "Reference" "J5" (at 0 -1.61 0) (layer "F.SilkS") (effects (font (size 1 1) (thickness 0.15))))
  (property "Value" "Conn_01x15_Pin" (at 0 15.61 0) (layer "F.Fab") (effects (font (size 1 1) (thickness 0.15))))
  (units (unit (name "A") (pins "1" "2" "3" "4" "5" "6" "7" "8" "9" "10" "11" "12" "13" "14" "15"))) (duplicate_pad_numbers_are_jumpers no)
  (pad "1" thru_hole rect (at 0 0) (size 0.85 0.85) (drill 0.5) (layers "*.Cu" "*.Mask") (remove_unused_layers no) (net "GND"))
  (pad "2" thru_hole circle (at 0 1) (size 0.85 0.85) (drill 0.5) (layers "*.Cu" "*.Mask") (remove_unused_layers no) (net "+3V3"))
  (pad "3" thru_hole circle (at 0 2) (size 0.85 0.85) (drill 0.5) (layers "*.Cu" "*.Mask") (remove_unused_layers no) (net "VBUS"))
  (pad "4" thru_hole circle (at 0 3) (size 0.85 0.85) (drill 0.5) (layers "*.Cu" "*.Mask") (remove_unused_layers no) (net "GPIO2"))
  (pad "5" thru_hole circle (at 0 4) (size 0.85 0.85) (drill 0.5) (layers "*.Cu" "*.Mask") (remove_unused_layers no) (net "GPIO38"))
  (pad "6" thru_hole circle (at 0 5) (size 0.85 0.85) (drill 0.5) (layers "*.Cu" "*.Mask") (remove_unused_layers no) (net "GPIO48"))
  (pad "7" thru_hole circle (at 0 6) (size 0.85 0.85) (drill 0.5) (layers "*.Cu" "*.Mask") (remove_unused_layers no) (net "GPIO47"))
  (pad "8" thru_hole circle (at 0 7) (size 0.85 0.85) (drill 0.5) (layers "*.Cu" "*.Mask") (remove_unused_layers no) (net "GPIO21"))
  (pad "9" thru_hole circle (at 0 8) (size 0.85 0.85) (drill 0.5) (layers "*.Cu" "*.Mask") (remove_unused_layers no) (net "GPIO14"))
  (pad "10" thru_hole circle (at 0 9) (size 0.85 0.85) (drill 0.5) (layers "*.Cu" "*.Mask") (remove_unused_layers no) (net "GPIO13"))
  (pad "11" thru_hole circle (at 0 10) (size 0.85 0.85) (drill 0.5) (layers "*.Cu" "*.Mask") (remove_unused_layers no) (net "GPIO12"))
  (pad "12" thru_hole circle (at 0 11) (size 0.85 0.85) (drill 0.5) (layers "*.Cu" "*.Mask") (remove_unused_layers no) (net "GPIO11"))
  (pad "13" thru_hole circle (at 0 12) (size 0.85 0.85) (drill 0.5) (layers "*.Cu" "*.Mask") (remove_unused_layers no) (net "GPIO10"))
  (pad "14" thru_hole circle (at 0 13) (size 0.85 0.85) (drill 0.5) (layers "*.Cu" "*.Mask") (remove_unused_layers no) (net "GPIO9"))
  (pad "15" thru_hole circle (at 0 14) (size 0.85 0.85) (drill 0.5) (layers "*.Cu" "*.Mask") (remove_unused_layers no) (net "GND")))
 (gr_rect (start 50 50) (end 79 95) (stroke (width 0.05) (type default)) (fill no) (layer "Edge.Cuts"))
 (segment (start 65.73241 86.93) (end 66 87.19759) (width 0.2) (layer "F.Cu") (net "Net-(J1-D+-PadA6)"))
 (segment (start 65 87.955) (end 65 87.19759) (width 0.2) (layer "F.Cu") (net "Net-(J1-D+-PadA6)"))
 (segment (start 65 87.19759) (end 65.26759 86.93) (width 0.2) (layer "F.Cu") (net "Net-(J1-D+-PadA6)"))
 (segment (start 65.26759 86.93) (end 65.73241 86.93) (width 0.2) (layer "F.Cu") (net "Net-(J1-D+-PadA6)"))
 (segment (start 66 87.19759) (end 66 87.955) (width 0.2) (layer "F.Cu") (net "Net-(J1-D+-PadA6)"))
 (segment (start 65.23241 88.98) (end 64.76759 88.98) (width 0.2) (layer "F.Cu") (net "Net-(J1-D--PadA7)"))
 (segment (start 65.5 88.71241) (end 65.23241 88.98) (width 0.2) (layer "F.Cu") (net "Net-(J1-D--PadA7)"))
 (segment (start 64.5 88.71241) (end 64.5 87.955) (width 0.2) (layer "F.Cu") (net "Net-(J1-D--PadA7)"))
 (segment (start 65.5 87.955) (end 65.5 88.71241) (width 0.2) (layer "F.Cu") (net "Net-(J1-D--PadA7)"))
 (segment (start 64.76759 88.98) (end 64.5 88.71241) (width 0.2) (layer "F.Cu") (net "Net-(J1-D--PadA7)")))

